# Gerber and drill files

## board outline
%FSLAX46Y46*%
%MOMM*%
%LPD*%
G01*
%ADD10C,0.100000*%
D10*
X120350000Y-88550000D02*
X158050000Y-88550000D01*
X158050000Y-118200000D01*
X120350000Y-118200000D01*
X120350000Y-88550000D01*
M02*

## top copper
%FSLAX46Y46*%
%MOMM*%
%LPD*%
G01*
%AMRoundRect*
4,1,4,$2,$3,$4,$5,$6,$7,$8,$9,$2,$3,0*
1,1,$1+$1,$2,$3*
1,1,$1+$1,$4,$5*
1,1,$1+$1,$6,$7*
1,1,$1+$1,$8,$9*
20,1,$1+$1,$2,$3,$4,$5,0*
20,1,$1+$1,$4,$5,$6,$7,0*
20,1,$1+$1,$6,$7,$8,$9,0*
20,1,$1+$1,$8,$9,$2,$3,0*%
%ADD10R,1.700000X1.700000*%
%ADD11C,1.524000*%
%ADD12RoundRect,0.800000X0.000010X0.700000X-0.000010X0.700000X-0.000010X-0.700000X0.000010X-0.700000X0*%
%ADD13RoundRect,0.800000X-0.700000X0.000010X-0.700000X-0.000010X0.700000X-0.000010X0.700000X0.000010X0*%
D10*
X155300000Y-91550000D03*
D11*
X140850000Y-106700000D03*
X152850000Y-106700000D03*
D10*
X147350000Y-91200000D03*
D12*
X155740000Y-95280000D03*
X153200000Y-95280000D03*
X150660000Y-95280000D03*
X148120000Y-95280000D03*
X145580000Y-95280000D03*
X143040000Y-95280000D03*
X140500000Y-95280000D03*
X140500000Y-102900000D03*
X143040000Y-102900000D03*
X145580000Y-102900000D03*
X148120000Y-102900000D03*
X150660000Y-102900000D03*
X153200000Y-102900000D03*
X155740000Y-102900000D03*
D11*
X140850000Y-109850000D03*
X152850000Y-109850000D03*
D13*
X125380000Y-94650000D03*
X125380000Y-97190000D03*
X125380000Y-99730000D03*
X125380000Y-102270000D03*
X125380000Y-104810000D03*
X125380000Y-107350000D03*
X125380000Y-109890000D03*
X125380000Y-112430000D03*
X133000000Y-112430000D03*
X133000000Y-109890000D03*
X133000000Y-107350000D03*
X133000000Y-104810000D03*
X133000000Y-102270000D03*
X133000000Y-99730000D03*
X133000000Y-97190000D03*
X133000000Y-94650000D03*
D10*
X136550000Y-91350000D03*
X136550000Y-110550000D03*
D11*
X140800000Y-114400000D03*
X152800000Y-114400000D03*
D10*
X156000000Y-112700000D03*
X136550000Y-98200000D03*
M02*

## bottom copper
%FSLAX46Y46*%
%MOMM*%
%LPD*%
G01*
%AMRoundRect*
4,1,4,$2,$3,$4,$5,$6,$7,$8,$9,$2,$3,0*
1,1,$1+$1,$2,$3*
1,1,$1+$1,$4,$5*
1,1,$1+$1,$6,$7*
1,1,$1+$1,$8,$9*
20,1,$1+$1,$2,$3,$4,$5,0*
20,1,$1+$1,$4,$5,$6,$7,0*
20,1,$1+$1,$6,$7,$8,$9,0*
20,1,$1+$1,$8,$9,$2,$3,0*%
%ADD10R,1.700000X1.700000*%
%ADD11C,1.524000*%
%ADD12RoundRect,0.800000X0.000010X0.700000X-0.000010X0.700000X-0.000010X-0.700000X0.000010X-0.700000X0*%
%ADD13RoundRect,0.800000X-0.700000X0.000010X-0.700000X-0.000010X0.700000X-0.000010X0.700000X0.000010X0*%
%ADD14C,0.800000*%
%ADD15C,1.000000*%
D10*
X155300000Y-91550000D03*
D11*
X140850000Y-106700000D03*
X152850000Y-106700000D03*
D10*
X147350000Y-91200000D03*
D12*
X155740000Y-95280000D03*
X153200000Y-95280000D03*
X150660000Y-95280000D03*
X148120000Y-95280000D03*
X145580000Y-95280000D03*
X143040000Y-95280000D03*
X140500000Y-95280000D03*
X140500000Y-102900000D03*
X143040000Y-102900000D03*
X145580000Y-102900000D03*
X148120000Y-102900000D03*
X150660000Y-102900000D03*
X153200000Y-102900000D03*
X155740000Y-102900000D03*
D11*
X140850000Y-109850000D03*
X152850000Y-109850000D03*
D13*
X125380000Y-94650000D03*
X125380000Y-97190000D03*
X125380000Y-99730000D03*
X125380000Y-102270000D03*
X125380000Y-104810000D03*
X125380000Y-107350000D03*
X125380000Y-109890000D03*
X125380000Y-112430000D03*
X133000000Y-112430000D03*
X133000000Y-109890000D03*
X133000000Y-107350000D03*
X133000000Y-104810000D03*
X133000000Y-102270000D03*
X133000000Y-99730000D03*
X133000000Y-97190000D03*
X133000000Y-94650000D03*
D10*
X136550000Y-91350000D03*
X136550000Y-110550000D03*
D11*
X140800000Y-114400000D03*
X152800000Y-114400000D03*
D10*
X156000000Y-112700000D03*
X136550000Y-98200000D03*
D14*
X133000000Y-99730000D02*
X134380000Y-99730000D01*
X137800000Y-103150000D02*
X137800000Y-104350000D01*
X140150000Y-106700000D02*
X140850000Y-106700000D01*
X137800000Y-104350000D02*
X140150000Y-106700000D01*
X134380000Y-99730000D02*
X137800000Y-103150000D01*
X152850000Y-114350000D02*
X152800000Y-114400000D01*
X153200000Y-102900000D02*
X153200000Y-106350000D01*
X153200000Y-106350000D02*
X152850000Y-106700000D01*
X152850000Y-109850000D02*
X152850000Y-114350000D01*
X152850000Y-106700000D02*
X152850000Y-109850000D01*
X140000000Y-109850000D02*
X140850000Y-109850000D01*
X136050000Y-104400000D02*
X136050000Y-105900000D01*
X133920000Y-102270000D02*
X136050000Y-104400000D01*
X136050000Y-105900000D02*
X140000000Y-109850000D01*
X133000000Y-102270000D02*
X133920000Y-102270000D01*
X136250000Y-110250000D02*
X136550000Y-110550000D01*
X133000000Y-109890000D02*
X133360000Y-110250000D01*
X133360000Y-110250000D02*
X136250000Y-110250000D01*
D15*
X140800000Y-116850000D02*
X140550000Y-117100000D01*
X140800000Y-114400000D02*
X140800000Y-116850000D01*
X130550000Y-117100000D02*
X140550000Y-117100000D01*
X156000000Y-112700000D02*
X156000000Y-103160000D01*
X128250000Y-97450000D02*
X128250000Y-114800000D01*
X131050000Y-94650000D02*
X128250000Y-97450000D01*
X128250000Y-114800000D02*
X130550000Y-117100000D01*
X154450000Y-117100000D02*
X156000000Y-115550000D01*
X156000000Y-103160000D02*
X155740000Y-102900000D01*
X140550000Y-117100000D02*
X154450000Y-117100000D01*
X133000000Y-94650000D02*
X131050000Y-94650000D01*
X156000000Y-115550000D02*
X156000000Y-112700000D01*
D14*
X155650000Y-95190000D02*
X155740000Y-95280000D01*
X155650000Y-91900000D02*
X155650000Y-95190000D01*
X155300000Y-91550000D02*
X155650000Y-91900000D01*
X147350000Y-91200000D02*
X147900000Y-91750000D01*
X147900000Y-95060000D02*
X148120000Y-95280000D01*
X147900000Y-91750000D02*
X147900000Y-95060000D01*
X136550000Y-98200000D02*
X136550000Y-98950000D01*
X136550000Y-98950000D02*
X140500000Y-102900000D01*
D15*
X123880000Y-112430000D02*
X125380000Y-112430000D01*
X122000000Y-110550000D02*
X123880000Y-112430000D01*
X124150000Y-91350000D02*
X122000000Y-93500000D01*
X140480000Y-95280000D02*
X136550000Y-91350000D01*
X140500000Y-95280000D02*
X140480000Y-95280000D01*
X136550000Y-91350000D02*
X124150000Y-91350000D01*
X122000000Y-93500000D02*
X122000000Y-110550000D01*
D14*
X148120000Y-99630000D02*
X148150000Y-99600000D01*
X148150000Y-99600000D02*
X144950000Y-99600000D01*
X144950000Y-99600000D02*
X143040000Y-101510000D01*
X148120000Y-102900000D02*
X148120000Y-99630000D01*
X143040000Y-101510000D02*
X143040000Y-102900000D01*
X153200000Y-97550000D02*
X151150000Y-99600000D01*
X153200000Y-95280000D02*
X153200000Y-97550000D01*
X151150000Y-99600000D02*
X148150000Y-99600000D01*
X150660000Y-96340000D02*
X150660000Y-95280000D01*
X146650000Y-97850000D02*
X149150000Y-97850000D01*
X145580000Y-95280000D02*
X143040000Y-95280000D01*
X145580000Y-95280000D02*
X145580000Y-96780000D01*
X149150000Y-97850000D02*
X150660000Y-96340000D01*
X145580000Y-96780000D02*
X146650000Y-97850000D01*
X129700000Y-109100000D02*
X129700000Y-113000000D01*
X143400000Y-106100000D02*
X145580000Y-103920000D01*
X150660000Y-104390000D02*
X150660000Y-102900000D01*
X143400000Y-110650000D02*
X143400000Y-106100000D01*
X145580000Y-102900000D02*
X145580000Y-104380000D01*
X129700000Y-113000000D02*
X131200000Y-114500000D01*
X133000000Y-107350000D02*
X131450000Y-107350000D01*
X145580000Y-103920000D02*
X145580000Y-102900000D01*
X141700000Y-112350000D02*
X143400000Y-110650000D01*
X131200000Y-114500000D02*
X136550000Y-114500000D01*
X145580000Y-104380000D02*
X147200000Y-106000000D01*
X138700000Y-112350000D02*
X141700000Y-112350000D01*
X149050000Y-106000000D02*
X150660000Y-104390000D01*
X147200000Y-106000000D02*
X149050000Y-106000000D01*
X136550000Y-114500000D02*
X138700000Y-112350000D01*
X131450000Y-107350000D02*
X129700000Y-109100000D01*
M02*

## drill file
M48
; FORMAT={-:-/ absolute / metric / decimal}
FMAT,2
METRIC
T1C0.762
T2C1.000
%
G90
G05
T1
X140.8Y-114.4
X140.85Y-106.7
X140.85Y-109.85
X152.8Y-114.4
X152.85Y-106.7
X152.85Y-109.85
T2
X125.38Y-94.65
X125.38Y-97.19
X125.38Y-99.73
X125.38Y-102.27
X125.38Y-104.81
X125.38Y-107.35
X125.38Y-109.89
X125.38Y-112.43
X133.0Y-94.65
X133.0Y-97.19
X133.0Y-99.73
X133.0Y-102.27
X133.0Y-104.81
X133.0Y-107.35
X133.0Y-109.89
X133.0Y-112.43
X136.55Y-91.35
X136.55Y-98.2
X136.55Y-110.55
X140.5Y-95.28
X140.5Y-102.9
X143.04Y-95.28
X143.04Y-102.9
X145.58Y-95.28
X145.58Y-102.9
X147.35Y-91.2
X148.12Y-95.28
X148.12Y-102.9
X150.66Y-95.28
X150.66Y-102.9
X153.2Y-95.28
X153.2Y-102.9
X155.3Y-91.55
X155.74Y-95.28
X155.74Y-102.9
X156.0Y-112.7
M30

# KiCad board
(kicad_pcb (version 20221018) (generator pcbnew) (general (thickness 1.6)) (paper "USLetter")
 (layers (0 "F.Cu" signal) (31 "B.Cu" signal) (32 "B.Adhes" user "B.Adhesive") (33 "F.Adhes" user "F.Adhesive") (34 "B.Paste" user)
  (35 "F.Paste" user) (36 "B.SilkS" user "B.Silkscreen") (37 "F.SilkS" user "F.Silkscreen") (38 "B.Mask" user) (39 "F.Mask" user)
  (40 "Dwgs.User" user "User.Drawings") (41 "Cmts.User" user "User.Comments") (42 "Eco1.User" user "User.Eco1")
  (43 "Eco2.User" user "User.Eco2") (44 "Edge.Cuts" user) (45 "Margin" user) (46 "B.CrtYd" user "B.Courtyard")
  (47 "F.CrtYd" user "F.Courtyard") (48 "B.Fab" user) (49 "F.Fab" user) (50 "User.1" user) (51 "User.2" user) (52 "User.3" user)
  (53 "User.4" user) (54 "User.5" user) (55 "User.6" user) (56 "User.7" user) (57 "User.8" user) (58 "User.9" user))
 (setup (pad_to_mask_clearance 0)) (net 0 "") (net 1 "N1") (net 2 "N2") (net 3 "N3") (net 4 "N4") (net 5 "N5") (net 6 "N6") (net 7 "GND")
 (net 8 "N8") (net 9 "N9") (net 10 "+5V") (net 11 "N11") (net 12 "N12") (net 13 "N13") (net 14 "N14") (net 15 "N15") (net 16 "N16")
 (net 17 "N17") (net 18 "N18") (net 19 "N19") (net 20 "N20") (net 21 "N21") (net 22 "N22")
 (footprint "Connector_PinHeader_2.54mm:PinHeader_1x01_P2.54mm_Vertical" (layer "F.Cu") (at 155.3 91.55)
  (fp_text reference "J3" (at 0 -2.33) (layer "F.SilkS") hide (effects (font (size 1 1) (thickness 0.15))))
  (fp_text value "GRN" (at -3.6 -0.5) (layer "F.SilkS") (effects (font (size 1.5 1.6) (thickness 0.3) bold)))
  (pad "1" thru_hole rect (at 0 0) (size 1.7 1.7) (drill 1) (layers "*.Cu" "*.Mask") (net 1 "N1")))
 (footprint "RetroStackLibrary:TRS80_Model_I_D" (layer "F.Cu") (at 146.85 106.7)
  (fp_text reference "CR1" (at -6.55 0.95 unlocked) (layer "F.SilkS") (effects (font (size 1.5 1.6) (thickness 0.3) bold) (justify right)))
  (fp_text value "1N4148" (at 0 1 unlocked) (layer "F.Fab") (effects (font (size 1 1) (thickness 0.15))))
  (pad "1" thru_hole circle (at -6 0) (size 1.524 1.524) (drill 0.762) (layers "*.Cu" "*.Mask") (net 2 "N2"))
  (pad "2" thru_hole circle (at 6 0) (size 1.524 1.524) (drill 0.762) (layers "*.Cu" "*.Mask") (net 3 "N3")))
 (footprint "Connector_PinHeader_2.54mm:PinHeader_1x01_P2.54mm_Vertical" (layer "F.Cu") (at 147.35 91.2)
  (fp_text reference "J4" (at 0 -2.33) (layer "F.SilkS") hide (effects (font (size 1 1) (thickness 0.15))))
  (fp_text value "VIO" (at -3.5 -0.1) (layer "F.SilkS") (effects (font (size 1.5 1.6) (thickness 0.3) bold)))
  (pad "1" thru_hole rect (at 0 0) (size 1.7 1.7) (drill 1) (layers "*.Cu" "*.Mask") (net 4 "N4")))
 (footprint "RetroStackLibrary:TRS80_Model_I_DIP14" (layer "F.Cu") (at 148.12 99.09 180)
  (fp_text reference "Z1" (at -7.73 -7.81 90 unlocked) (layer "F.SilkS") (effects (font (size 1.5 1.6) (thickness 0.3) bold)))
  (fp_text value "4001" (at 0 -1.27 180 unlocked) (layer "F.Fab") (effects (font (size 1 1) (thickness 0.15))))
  (pad "1" thru_hole roundrect (at -7.62 3.81 180) (size 1.6 3) (drill 1) (layers "*.Cu" "*.Mask") (roundrect_rratio 0.5) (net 1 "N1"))
  (pad "2" thru_hole roundrect (at -5.08 3.81 180) (size 1.6 3) (drill 1) (layers "*.Cu" "*.Mask") (roundrect_rratio 0.5) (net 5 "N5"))
  (pad "3" thru_hole roundrect (at -2.54 3.81 180) (size 1.6 3) (drill 1) (layers "*.Cu" "*.Mask") (roundrect_rratio 0.5) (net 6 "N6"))
  (pad "4" thru_hole roundrect (at 0 3.81 180) (size 1.6 3) (drill 1) (layers "*.Cu" "*.Mask") (roundrect_rratio 0.5) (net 4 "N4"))
  (pad "5" thru_hole roundrect (at 2.54 3.81 180) (size 1.6 3) (drill 1) (layers "*.Cu" "*.Mask") (roundrect_rratio 0.5) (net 6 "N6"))
  (pad "6" thru_hole roundrect (at 5.08 3.81 180) (size 1.6 3) (drill 1) (layers "*.Cu" "*.Mask") (roundrect_rratio 0.5) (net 6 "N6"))
  (pad "7" thru_hole roundrect (at 7.62 3.81 180) (size 1.6 3) (drill 1) (layers "*.Cu" "*.Mask") (roundrect_rratio 0.5) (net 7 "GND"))
  (pad "8" thru_hole roundrect (at 7.62 -3.81 180) (size 1.6 3) (drill 1) (layers "*.Cu" "*.Mask") (roundrect_rratio 0.5) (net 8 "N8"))
  (pad "9" thru_hole roundrect (at 5.08 -3.81 180) (size 1.6 3) (drill 1) (layers "*.Cu" "*.Mask") (roundrect_rratio 0.5) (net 5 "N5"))
  (pad "10" thru_hole roundrect (at 2.54 -3.81 180) (size 1.6 3) (drill 1) (layers "*.Cu" "*.Mask") (roundrect_rratio 0.5) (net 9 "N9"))
  (pad "11" thru_hole roundrect (at 0 -3.81 180) (size 1.6 3) (drill 1) (layers "*.Cu" "*.Mask") (roundrect_rratio 0.5) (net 5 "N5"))
  (pad "12" thru_hole roundrect (at -2.54 -3.81 180) (size 1.6 3) (drill 1) (layers "*.Cu" "*.Mask") (roundrect_rratio 0.5) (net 9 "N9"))
  (pad "13" thru_hole roundrect (at -5.08 -3.81 180) (size 1.6 3) (drill 1) (layers "*.Cu" "*.Mask") (roundrect_rratio 0.5) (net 3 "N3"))
  (pad "14" thru_hole roundrect (at -7.62 -3.81 180) (size 1.6 3) (drill 1) (layers "*.Cu" "*.Mask") (roundrect_rratio 0.5) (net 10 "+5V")))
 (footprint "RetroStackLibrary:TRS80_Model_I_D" (layer "F.Cu") (at 146.85 109.85)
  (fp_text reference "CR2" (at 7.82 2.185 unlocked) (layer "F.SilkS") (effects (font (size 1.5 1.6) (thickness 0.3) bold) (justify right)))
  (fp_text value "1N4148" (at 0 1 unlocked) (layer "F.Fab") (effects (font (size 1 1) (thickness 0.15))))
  (pad "1" thru_hole circle (at -6 0) (size 1.524 1.524) (drill 0.762) (layers "*.Cu" "*.Mask") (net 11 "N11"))
  (pad "2" thru_hole circle (at 6 0) (size 1.524 1.524) (drill 0.762) (layers "*.Cu" "*.Mask") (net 3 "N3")))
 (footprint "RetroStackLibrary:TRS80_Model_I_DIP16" (layer "F.Cu") (at 129.19 103.54 -90)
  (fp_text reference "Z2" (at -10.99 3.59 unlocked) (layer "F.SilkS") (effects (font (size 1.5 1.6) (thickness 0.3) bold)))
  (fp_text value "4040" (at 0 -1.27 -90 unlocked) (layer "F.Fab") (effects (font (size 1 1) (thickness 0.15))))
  (pad "1" thru_hole roundrect (at -8.89 3.81 270) (size 1.6 3) (drill 1) (layers "*.Cu" "*.Mask") (roundrect_rratio 0.5) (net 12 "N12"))
  (pad "2" thru_hole roundrect (at -6.35 3.81 270) (size 1.6 3) (drill 1) (layers "*.Cu" "*.Mask") (roundrect_rratio 0.5) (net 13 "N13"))
  (pad "3" thru_hole roundrect (at -3.81 3.81 270) (size 1.6 3) (drill 1) (layers "*.Cu" "*.Mask") (roundrect_rratio 0.5) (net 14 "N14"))
  (pad "4" thru_hole roundrect (at -1.27 3.81 270) (size 1.6 3) (drill 1) (layers "*.Cu" "*.Mask") (roundrect_rratio 0.5) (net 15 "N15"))
  (pad "5" thru_hole roundrect (at 1.27 3.81 270) (size 1.6 3) (drill 1) (layers "*.Cu" "*.Mask") (roundrect_rratio 0.5) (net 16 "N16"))
  (pad "6" thru_hole roundrect (at 3.81 3.81 270) (size 1.6 3) (drill 1) (layers "*.Cu" "*.Mask") (roundrect_rratio 0.5) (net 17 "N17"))
  (pad "7" thru_hole roundrect (at 6.35 3.81 270) (size 1.6 3) (drill 1) (layers "*.Cu" "*.Mask") (roundrect_rratio 0.5) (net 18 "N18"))
  (pad "8" thru_hole roundrect (at 8.89 3.81 270) (size 1.6 3) (drill 1) (layers "*.Cu" "*.Mask") (roundrect_rratio 0.5) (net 7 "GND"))
  (pad "9" thru_hole roundrect (at 8.89 -3.81 270) (size 1.6 3) (drill 1) (layers "*.Cu" "*.Mask") (roundrect_rratio 0.5) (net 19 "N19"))
  (pad "10" thru_hole roundrect (at 6.35 -3.81 270) (size 1.6 3) (drill 1) (layers "*.Cu" "*.Mask") (roundrect_rratio 0.5) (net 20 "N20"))
  (pad "11" thru_hole roundrect (at 3.81 -3.81 270) (size 1.6 3) (drill 1) (layers "*.Cu" "*.Mask") (roundrect_rratio 0.5) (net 9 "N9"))
  (pad "12" thru_hole roundrect (at 1.27 -3.81 270) (size 1.6 3) (drill 1) (layers "*.Cu" "*.Mask") (roundrect_rratio 0.5) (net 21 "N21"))
  (pad "13" thru_hole roundrect (at -1.27 -3.81 270) (size 1.6 3) (drill 1) (layers "*.Cu" "*.Mask") (roundrect_rratio 0.5) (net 11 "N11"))
  (pad "14" thru_hole roundrect (at -3.81 -3.81 270) (size 1.6 3) (drill 1) (layers "*.Cu" "*.Mask") (roundrect_rratio 0.5) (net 2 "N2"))
  (pad "15" thru_hole roundrect (at -6.35 -3.81 270) (size 1.6 3) (drill 1) (layers "*.Cu" "*.Mask") (roundrect_rratio 0.5) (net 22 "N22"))
  (pad "16" thru_hole roundrect (at -8.89 -3.81 270) (size 1.6 3) (drill 1) (layers "*.Cu" "*.Mask") (roundrect_rratio 0.5) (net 10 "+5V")))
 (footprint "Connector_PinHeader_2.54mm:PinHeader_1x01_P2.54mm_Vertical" (layer "F.Cu") (at 136.55 91.35)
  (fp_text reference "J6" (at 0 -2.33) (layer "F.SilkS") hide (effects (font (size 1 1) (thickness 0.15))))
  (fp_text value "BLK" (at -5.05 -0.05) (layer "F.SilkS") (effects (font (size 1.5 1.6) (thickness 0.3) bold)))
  (pad "1" thru_hole rect (at 0 0) (size 1.7 1.7) (drill 1) (layers "*.Cu" "*.Mask") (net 7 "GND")))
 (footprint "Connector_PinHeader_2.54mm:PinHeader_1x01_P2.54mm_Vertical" (layer "F.Cu") (at 136.55 110.55)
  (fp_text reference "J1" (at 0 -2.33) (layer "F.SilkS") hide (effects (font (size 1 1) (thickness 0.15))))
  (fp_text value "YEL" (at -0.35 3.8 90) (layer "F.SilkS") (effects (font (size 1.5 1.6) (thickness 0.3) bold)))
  (pad "1" thru_hole rect (at 0 0) (size 1.7 1.7) (drill 1) (layers "*.Cu" "*.Mask") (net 20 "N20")))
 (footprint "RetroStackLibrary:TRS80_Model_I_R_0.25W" (layer "F.Cu") (at 146.8 114.4)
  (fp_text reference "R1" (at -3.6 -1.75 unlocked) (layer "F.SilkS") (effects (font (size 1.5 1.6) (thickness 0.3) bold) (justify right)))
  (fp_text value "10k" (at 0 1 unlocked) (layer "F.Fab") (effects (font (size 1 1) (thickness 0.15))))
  (pad "1" thru_hole circle (at -6 0) (size 1.524 1.524) (drill 0.762) (layers "*.Cu" "*.Mask") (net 10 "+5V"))
  (pad "2" thru_hole circle (at 6 0) (size 1.524 1.524) (drill 0.762) (layers "*.Cu" "*.Mask") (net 3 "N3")))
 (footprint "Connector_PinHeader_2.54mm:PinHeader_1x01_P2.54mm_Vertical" (layer "F.Cu") (at 156 112.7)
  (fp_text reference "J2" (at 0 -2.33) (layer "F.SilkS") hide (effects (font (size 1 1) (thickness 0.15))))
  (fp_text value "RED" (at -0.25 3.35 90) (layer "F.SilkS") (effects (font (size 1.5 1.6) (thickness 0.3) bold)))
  (pad "1" thru_hole rect (at 0 0) (size 1.7 1.7) (drill 1) (layers "*.Cu" "*.Mask") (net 10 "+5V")))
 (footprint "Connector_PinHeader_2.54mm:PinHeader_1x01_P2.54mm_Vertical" (layer "F.Cu") (at 136.55 98.2)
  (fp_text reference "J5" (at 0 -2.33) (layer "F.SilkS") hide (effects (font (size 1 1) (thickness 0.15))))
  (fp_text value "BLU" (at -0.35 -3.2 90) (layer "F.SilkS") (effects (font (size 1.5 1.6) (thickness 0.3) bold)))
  (pad "1" thru_hole rect (at 0 0) (size 1.7 1.7) (drill 1) (layers "*.Cu" "*.Mask") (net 8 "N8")))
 (gr_rect (start 120.35 88.55) (end 158.05 118.2) (stroke (width 0.1) (type default)) (fill none) (layer "Edge.Cuts"))
 (segment (start 133 99.73) (end 134.38 99.73) (width 0.8) (layer "B.Cu") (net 2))
 (segment (start 137.8 103.15) (end 137.8 104.35) (width 0.8) (layer "B.Cu") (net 2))
 (segment (start 140.15 106.7) (end 140.85 106.7) (width 0.8) (layer "B.Cu") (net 2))
 (segment (start 137.8 104.35) (end 140.15 106.7) (width 0.8) (layer "B.Cu") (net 2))
 (segment (start 134.38 99.73) (end 137.8 103.15) (width 0.8) (layer "B.Cu") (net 2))
 (segment (start 152.85 114.35) (end 152.8 114.4) (width 0.8) (layer "B.Cu") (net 3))
 (segment (start 153.2 102.9) (end 153.2 106.35) (width 0.8) (layer "B.Cu") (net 3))
 (segment (start 153.2 106.35) (end 152.85 106.7) (width 0.8) (layer "B.Cu") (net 3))
 (segment (start 152.85 109.85) (end 152.85 114.35) (width 0.8) (layer "B.Cu") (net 3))
 (segment (start 152.85 106.7) (end 152.85 109.85) (width 0.8) (layer "B.Cu") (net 3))
 (segment (start 140 109.85) (end 140.85 109.85) (width 0.8) (layer "B.Cu") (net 11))
 (segment (start 136.05 104.4) (end 136.05 105.9) (width 0.8) (layer "B.Cu") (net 11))
 (segment (start 133.92 102.27) (end 136.05 104.4) (width 0.8) (layer "B.Cu") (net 11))
 (segment (start 136.05 105.9) (end 140 109.85) (width 0.8) (layer "B.Cu") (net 11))
 (segment (start 133 102.27) (end 133.92 102.27) (width 0.8) (layer "B.Cu") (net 11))
 (segment (start 136.25 110.25) (end 136.55 110.55) (width 0.8) (layer "B.Cu") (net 20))
 (segment (start 133 109.89) (end 133.36 110.25) (width 0.8) (layer "B.Cu") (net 20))
 (segment (start 133.36 110.25) (end 136.25 110.25) (width 0.8) (layer "B.Cu") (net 20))
 (segment (start 140.8 116.85) (end 140.55 117.1) (width 1) (layer "B.Cu") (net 10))
 (segment (start 140.8 114.4) (end 140.8 116.85) (width 1) (layer "B.Cu") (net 10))
 (segment (start 130.55 117.1) (end 140.55 117.1) (width 1) (layer "B.Cu") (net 10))
 (segment (start 156 112.7) (end 156 103.16) (width 1) (layer "B.Cu") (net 10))
 (segment (start 128.25 97.45) (end 128.25 114.8) (width 1) (layer "B.Cu") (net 10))
 (segment (start 131.05 94.65) (end 128.25 97.45) (width 1) (layer "B.Cu") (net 10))
 (segment (start 128.25 114.8) (end 130.55 117.1) (width 1) (layer "B.Cu") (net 10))
 (segment (start 154.45 117.1) (end 156 115.55) (width 1) (layer "B.Cu") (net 10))
 (segment (start 156 103.16) (end 155.74 102.9) (width 1) (layer "B.Cu") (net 10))
 (segment (start 140.55 117.1) (end 154.45 117.1) (width 1) (layer "B.Cu") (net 10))
 (segment (start 133 94.65) (end 131.05 94.65) (width 1) (layer "B.Cu") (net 10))
 (segment (start 156 115.55) (end 156 112.7) (width 1) (layer "B.Cu") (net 10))
 (segment (start 155.65 95.19) (end 155.74 95.28) (width 0.8) (layer "B.Cu") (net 1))
 (segment (start 155.65 91.9) (end 155.65 95.19) (width 0.8) (layer "B.Cu") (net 1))
 (segment (start 155.3 91.55) (end 155.65 91.9) (width 0.8) (layer "B.Cu") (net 1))
 (segment (start 147.35 91.2) (end 147.9 91.75) (width 0.8) (layer "B.Cu") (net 4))
 (segment (start 147.9 95.06) (end 148.12 95.28) (width 0.8) (layer "B.Cu") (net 4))
 (segment (start 147.9 91.75) (end 147.9 95.06) (width 0.8) (layer "B.Cu") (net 4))
 (segment (start 136.55 98.2) (end 136.55 98.95) (width 0.8) (layer "B.Cu") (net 8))
 (segment (start 136.55 98.95) (end 140.5 102.9) (width 0.8) (layer "B.Cu") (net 8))
 (segment (start 123.88 112.43) (end 125.38 112.43) (width 1) (layer "B.Cu") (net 7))
 (segment (start 122 110.55) (end 123.88 112.43) (width 1) (layer "B.Cu") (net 7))
 (segment (start 124.15 91.35) (end 122 93.5) (width 1) (layer "B.Cu") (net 7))
 (segment (start 140.48 95.28) (end 136.55 91.35) (width 1) (layer "B.Cu") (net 7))
 (segment (start 140.5 95.28) (end 140.48 95.28) (width 1) (layer "B.Cu") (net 7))
 (segment (start 136.55 91.35) (end 124.15 91.35) (width 1) (layer "B.Cu") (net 7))
 (segment (start 122 93.5) (end 122 110.55) (width 1) (layer "B.Cu") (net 7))
 (segment (start 148.12 99.63) (end 148.15 99.6) (width 0.8) (layer "B.Cu") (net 5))
 (segment (start 148.15 99.6) (end 144.95 99.6) (width 0.8) (layer "B.Cu") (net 5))
 (segment (start 144.95 99.6) (end 143.04 101.51) (width 0.8) (layer "B.Cu") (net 5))
 (segment (start 148.12 102.9) (end 148.12 99.63) (width 0.8) (layer "B.Cu") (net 5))
 (segment (start 143.04 101.51) (end 143.04 102.9) (width 0.8) (layer "B.Cu") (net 5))
 (segment (start 153.2 97.55) (end 151.15 99.6) (width 0.8) (layer "B.Cu") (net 5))
 (segment (start 153.2 95.28) (end 153.2 97.55) (width 0.8) (layer "B.Cu") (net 5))
 (segment (start 151.15 99.6) (end 148.15 99.6) (width 0.8) (layer "B.Cu") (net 5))
 (segment (start 150.66 96.34) (end 150.66 95.28) (width 0.8) (layer "B.Cu") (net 6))
 (segment (start 146.65 97.85) (end 149.15 97.85) (width 0.8) (layer "B.Cu") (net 6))
 (segment (start 145.58 95.28) (end 143.04 95.28) (width 0.8) (layer "B.Cu") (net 6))
 (segment (start 145.58 95.28) (end 145.58 96.78) (width 0.8) (layer "B.Cu") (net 6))
 (segment (start 149.15 97.85) (end 150.66 96.34) (width 0.8) (layer "B.Cu") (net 6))
 (segment (start 145.58 96.78) (end 146.65 97.85) (width 0.8) (layer "B.Cu") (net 6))
 (segment (start 129.7 109.1) (end 129.7 113) (width 0.8) (layer "B.Cu") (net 9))
 (segment (start 143.4 106.1) (end 145.58 103.92) (width 0.8) (layer "B.Cu") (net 9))
 (segment (start 150.66 104.39) (end 150.66 102.9) (width 0.8) (layer "B.Cu") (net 9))
 (segment (start 143.4 110.65) (end 143.4 106.1) (width 0.8) (layer "B.Cu") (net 9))
 (segment (start 145.58 102.9) (end 145.58 104.38) (width 0.8) (layer "B.Cu") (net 9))
 (segment (start 129.7 113) (end 131.2 114.5) (width 0.8) (layer "B.Cu") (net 9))
 (segment (start 133 107.35) (end 131.45 107.35) (width 0.8) (layer "B.Cu") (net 9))
 (segment (start 145.58 103.92) (end 145.58 102.9) (width 0.8) (layer "B.Cu") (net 9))
 (segment (start 141.7 112.35) (end 143.4 110.65) (width 0.8) (layer "B.Cu") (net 9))
 (segment (start 131.2 114.5) (end 136.55 114.5) (width 0.8) (layer "B.Cu") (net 9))
 (segment (start 145.58 104.38) (end 147.2 106) (width 0.8) (layer "B.Cu") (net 9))
 (segment (start 138.7 112.35) (end 141.7 112.35) (width 0.8) (layer "B.Cu") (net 9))
 (segment (start 149.05 106) (end 150.66 104.39) (width 0.8) (layer "B.Cu") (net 9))
 (segment (start 147.2 106) (end 149.05 106) (width 0.8) (layer "B.Cu") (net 9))
 (segment (start 136.55 114.5) (end 138.7 112.35) (width 0.8) (layer "B.Cu") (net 9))
 (segment (start 131.45 107.35) (end 129.7 109.1) (width 0.8) (layer "B.Cu") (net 9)))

